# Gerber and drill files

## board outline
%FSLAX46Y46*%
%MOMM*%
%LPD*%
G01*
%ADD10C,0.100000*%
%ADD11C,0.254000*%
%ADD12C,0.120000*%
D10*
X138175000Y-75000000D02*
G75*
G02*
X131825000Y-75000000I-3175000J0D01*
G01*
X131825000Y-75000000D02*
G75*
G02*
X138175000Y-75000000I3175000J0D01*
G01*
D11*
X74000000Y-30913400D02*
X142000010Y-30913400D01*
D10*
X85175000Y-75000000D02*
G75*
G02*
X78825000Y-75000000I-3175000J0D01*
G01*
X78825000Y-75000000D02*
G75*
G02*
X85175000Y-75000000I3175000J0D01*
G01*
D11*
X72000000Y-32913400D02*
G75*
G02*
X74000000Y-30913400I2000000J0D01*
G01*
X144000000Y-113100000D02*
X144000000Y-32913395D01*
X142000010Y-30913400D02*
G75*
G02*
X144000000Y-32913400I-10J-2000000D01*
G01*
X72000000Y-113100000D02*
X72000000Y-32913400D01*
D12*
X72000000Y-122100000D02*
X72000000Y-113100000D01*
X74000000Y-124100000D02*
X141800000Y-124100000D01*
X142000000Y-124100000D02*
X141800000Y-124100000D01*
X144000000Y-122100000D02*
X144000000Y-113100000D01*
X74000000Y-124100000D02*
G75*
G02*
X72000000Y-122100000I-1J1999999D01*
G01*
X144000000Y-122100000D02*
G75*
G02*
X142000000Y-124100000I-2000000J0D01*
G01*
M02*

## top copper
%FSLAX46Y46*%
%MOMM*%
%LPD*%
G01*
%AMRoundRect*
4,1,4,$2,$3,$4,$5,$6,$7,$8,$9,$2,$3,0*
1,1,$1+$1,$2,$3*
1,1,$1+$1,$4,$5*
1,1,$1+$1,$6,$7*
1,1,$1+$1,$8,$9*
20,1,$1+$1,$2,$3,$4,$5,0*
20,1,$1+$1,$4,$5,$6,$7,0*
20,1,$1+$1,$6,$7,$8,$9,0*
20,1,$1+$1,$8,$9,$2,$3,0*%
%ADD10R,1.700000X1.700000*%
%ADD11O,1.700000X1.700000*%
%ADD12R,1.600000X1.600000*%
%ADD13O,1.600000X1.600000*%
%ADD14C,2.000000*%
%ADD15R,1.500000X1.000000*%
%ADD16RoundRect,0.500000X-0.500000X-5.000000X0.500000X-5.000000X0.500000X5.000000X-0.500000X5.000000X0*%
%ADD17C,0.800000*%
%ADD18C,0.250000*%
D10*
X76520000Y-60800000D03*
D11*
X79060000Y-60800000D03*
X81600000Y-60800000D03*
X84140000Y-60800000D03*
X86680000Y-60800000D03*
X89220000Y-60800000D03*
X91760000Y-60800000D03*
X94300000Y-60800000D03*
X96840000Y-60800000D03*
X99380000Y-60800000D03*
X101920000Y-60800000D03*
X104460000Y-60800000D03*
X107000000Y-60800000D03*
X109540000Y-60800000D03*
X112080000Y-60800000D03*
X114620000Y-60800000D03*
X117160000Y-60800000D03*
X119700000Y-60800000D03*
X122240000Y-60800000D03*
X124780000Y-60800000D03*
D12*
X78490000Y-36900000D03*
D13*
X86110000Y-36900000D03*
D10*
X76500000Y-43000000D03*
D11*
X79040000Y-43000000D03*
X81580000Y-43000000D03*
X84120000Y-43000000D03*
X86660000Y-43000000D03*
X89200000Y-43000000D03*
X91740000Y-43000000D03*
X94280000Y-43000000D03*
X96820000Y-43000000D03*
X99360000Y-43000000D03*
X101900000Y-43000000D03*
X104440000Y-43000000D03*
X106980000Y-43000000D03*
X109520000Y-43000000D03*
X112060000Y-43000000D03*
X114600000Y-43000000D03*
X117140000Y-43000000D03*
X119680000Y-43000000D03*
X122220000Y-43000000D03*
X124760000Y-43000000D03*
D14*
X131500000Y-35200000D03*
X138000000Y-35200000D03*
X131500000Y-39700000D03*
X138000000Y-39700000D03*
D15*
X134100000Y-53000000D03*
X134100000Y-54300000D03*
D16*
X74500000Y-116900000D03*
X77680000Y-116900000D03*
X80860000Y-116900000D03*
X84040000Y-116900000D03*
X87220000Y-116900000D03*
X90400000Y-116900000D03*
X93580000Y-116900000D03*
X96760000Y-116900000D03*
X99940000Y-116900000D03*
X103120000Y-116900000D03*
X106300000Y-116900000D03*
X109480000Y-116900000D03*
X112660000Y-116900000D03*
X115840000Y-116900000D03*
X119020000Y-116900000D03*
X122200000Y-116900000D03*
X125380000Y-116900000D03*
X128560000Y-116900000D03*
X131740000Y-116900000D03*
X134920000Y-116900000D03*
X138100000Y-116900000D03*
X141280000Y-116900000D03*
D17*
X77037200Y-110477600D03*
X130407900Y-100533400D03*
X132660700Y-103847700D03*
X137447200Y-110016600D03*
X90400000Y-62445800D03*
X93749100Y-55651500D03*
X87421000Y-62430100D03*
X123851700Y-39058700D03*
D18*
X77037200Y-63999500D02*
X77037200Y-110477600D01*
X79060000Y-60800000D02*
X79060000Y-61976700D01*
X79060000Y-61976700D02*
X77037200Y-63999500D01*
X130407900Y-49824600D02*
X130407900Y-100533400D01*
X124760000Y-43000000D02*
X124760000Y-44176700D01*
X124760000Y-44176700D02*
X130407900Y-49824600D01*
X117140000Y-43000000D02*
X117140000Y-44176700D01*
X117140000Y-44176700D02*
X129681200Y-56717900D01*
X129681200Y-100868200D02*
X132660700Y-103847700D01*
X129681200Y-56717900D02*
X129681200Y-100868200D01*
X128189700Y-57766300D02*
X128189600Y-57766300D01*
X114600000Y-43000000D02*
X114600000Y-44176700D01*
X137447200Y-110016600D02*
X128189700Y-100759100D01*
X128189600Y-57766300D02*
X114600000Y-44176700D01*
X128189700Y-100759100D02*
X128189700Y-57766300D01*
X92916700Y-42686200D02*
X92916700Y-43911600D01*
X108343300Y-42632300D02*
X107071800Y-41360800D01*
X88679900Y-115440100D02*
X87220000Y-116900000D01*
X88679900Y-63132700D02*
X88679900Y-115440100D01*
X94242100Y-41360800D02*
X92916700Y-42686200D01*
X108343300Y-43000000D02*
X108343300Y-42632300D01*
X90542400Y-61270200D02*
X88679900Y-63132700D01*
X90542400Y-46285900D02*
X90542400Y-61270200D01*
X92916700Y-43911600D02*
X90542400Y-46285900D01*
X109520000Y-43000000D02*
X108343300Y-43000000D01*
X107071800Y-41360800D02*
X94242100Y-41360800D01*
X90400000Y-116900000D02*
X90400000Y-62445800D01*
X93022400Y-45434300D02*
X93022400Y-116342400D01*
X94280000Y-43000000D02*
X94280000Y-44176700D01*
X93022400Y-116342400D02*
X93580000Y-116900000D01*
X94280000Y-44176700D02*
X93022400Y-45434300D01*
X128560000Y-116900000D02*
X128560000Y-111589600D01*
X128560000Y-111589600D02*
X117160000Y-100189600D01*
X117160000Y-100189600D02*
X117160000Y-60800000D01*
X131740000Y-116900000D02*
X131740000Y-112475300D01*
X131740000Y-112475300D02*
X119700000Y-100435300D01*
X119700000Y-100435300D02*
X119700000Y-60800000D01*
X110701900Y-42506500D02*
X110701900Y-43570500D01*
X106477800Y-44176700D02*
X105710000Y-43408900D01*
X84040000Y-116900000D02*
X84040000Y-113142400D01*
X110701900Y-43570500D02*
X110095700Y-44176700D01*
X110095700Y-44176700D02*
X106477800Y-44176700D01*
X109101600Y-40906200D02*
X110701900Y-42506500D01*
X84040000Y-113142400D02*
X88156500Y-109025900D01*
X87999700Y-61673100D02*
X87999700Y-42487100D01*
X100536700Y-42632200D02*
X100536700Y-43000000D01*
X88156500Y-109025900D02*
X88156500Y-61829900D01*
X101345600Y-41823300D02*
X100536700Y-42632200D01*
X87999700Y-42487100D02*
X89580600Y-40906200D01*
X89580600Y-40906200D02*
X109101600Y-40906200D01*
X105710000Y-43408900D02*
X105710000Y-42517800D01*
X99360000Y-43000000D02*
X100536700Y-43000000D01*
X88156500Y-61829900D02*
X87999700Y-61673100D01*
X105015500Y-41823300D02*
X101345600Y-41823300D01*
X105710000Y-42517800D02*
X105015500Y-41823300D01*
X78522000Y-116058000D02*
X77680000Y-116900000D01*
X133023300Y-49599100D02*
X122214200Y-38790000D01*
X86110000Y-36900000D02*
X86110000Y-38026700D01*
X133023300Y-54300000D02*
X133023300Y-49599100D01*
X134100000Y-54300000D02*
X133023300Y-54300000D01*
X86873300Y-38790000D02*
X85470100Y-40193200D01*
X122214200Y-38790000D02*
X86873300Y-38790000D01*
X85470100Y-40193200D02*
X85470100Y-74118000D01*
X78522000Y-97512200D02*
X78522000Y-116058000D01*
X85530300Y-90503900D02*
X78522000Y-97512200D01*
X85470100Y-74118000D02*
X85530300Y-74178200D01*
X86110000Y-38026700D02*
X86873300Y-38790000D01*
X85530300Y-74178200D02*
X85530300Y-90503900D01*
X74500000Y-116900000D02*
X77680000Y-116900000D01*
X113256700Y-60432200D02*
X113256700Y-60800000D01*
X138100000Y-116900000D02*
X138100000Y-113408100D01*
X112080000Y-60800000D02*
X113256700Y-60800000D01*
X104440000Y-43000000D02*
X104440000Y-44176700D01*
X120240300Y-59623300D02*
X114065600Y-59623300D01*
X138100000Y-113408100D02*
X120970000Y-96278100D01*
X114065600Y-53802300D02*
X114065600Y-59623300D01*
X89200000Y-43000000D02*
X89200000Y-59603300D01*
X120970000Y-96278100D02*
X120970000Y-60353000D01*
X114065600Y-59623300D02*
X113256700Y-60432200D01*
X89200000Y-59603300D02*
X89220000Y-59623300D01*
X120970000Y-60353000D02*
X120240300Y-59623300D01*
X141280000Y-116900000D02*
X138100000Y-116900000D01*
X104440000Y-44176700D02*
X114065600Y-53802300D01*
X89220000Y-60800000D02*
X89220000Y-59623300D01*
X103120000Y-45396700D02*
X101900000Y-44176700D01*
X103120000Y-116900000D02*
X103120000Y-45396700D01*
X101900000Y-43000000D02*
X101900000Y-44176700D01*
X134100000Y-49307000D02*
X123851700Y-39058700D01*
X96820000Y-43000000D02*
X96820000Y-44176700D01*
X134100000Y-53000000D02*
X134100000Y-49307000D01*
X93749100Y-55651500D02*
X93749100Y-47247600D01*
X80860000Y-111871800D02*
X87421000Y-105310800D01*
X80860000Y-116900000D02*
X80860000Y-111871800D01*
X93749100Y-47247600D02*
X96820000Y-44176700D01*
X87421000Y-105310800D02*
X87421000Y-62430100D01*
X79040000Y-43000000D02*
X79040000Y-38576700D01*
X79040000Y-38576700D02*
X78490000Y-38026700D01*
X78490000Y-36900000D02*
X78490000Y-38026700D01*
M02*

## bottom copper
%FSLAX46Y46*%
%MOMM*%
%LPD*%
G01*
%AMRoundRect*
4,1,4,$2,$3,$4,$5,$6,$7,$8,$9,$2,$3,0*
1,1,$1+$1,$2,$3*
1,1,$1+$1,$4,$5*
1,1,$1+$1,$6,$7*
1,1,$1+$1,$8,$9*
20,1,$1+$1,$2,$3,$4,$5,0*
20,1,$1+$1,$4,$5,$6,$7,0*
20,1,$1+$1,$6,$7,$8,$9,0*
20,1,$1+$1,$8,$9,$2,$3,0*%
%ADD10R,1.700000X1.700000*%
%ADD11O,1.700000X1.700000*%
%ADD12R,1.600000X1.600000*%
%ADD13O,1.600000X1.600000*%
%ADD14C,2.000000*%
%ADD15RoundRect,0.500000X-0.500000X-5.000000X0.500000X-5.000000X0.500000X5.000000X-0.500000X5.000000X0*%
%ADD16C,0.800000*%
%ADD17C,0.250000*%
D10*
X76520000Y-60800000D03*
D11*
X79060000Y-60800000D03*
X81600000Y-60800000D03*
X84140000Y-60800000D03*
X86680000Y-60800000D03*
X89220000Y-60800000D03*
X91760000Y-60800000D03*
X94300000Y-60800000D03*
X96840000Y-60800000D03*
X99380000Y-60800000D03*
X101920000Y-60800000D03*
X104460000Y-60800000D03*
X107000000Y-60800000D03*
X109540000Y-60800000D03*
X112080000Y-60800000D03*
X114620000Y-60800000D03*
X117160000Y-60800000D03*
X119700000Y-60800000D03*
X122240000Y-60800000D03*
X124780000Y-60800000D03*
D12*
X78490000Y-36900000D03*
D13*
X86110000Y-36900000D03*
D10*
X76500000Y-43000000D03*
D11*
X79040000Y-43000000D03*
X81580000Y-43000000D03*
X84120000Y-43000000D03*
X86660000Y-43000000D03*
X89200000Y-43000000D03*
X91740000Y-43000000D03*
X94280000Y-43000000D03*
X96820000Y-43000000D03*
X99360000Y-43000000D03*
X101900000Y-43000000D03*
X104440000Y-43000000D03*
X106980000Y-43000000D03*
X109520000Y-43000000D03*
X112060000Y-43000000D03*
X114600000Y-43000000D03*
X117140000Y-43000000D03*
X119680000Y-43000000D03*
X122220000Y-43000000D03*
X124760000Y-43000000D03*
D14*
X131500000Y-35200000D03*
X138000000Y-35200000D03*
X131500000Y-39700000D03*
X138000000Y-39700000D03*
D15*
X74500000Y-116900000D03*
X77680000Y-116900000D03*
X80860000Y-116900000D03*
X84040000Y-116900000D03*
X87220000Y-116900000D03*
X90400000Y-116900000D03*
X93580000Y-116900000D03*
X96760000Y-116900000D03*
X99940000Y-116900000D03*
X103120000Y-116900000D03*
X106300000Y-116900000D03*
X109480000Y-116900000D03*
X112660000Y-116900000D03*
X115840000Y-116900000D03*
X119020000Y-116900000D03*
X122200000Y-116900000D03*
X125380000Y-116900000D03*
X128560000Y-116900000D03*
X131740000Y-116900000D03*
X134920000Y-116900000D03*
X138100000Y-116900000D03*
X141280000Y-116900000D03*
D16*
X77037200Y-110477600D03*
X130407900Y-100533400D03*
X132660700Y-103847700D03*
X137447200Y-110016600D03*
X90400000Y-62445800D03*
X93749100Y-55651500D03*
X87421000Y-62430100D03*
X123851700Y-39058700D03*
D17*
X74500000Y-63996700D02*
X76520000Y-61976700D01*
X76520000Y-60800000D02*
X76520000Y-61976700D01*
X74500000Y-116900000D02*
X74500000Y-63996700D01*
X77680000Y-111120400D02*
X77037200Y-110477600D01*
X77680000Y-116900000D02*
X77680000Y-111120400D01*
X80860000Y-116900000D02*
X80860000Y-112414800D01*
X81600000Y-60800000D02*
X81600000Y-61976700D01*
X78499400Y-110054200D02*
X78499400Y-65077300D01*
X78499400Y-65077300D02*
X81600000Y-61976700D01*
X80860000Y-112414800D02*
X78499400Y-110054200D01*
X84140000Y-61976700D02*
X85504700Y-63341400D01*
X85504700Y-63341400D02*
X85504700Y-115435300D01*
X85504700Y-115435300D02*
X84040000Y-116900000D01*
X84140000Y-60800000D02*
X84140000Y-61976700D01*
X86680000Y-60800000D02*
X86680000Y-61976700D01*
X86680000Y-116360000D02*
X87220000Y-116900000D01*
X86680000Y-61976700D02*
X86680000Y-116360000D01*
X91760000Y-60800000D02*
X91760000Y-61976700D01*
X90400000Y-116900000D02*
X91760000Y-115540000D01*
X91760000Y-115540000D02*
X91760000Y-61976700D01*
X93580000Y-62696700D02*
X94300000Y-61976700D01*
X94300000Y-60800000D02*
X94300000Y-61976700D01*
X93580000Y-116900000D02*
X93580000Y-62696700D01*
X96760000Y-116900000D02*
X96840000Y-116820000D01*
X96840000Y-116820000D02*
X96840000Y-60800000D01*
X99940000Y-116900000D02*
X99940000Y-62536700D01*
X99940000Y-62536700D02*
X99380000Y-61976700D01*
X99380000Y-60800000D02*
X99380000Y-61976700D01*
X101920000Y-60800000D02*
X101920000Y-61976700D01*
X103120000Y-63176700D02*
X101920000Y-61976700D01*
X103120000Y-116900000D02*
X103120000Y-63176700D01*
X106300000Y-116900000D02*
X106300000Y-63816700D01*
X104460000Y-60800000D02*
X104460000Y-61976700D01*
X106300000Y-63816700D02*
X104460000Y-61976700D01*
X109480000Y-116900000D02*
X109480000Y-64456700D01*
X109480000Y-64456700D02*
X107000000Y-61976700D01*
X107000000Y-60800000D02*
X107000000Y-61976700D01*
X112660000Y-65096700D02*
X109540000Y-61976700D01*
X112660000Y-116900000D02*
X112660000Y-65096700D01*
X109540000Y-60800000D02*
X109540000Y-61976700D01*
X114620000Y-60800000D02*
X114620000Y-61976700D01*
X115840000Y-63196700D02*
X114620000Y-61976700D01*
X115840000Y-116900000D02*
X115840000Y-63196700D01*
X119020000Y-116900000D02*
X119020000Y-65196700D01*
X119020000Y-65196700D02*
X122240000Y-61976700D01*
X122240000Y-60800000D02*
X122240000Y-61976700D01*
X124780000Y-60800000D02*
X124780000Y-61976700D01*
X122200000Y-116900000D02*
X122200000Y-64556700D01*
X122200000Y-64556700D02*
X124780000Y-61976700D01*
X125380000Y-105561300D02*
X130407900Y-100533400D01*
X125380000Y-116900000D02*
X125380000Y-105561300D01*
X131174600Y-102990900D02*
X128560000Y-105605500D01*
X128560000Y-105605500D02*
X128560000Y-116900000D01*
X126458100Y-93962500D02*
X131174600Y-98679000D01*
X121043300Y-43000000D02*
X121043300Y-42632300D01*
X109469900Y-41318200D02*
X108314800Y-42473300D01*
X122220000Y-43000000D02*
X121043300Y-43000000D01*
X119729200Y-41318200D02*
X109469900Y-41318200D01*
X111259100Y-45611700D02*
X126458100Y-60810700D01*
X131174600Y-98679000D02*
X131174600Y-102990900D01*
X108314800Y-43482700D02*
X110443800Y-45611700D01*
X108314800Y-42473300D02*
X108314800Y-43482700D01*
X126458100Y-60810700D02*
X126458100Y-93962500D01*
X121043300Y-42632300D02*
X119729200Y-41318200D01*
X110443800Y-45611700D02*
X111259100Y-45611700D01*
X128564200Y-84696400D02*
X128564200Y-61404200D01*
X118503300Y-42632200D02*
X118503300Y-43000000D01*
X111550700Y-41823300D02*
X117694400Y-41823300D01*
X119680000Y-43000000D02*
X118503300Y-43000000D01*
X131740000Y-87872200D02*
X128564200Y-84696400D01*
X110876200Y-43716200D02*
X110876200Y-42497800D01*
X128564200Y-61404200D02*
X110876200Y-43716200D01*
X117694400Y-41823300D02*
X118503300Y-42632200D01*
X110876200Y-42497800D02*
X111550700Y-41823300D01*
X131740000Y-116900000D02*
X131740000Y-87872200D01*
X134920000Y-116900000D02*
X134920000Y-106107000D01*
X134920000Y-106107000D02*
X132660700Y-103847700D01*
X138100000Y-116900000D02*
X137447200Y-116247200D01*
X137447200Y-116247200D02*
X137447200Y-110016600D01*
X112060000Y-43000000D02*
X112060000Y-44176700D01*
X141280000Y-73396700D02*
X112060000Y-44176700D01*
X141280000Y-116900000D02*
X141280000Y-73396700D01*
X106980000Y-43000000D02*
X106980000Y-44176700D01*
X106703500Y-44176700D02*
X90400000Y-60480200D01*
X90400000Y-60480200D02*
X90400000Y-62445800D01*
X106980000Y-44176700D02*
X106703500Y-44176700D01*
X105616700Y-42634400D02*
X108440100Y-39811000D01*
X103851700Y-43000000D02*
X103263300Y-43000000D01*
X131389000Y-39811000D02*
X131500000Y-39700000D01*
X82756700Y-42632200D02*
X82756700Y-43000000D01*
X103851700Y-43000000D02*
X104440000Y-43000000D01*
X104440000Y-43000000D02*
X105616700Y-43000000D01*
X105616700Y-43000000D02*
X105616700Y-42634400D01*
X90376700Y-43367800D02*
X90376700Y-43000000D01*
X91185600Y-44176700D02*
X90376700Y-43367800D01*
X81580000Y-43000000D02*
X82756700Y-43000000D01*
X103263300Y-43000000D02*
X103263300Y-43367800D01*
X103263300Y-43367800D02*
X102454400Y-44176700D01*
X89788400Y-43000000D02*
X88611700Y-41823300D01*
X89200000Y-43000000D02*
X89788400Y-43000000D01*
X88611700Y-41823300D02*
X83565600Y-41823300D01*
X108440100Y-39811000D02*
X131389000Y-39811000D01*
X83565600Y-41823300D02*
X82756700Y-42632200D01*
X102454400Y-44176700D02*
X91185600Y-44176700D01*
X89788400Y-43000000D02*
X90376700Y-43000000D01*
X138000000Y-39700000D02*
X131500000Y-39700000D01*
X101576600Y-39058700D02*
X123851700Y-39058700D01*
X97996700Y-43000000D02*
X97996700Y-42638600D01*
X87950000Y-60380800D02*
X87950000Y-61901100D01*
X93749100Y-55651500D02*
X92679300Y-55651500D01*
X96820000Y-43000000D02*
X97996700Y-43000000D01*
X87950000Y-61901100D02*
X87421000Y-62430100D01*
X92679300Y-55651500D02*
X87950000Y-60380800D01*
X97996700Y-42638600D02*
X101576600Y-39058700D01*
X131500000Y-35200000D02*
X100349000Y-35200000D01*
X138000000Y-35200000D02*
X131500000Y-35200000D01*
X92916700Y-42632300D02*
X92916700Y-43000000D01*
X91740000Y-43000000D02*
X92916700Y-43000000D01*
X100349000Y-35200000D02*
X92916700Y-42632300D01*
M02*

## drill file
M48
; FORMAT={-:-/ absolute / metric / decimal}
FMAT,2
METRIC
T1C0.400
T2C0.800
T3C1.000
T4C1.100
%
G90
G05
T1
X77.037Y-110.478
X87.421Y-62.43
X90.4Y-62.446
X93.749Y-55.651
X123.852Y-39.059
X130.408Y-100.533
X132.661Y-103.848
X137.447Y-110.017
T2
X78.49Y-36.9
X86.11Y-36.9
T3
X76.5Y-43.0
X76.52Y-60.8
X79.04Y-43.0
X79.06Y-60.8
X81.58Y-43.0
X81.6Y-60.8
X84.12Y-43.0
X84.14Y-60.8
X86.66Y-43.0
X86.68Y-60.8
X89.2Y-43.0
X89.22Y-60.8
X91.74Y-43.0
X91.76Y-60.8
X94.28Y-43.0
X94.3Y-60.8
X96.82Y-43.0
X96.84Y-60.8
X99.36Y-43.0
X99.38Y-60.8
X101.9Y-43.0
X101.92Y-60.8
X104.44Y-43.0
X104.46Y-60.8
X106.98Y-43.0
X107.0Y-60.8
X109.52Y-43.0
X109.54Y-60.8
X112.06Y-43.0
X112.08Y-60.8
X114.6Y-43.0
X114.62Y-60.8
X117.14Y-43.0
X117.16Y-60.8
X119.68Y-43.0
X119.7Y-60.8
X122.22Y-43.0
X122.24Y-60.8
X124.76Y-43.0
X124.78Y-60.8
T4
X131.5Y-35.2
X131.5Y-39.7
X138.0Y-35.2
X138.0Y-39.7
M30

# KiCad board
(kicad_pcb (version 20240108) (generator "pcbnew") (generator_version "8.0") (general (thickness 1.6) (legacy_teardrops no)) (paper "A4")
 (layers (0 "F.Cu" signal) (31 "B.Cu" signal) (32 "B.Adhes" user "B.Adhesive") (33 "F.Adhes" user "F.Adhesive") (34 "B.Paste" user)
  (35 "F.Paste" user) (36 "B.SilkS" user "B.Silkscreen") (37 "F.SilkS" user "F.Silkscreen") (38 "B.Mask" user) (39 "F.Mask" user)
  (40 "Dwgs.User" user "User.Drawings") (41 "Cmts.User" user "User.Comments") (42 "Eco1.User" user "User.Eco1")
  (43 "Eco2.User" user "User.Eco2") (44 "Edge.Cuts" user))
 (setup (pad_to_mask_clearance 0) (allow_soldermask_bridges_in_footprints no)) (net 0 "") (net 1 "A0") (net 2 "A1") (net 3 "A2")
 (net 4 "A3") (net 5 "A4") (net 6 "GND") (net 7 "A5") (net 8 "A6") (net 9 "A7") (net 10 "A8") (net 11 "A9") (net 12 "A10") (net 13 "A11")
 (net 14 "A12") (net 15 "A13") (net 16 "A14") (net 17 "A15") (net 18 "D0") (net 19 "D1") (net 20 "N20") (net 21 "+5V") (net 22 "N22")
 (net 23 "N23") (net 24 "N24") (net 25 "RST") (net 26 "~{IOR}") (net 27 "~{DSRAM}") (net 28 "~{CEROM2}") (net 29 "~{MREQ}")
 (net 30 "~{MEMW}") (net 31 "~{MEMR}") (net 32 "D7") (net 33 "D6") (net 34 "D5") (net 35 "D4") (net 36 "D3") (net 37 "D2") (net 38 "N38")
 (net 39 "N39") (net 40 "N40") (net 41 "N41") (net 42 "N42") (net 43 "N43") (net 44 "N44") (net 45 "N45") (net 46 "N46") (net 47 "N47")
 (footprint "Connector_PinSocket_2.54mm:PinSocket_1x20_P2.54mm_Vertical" (layer "F.Cu") (at 76.52 60.8 90)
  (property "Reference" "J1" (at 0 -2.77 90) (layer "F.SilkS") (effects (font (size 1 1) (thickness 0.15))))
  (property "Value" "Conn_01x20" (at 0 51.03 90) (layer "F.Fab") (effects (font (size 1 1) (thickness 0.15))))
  (pad "1" thru_hole rect (at 0 0 90) (size 1.7 1.7) (drill 1) (layers "*.Cu" "*.Mask") (remove_unused_layers no) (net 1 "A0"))
  (pad "2" thru_hole oval (at 0 2.54 90) (size 1.7 1.7) (drill 1) (layers "*.Cu" "*.Mask") (remove_unused_layers no) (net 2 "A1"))
  (pad "3" thru_hole oval (at 0 5.08 90) (size 1.7 1.7) (drill 1) (layers "*.Cu" "*.Mask") (remove_unused_layers no) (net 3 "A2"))
  (pad "4" thru_hole oval (at 0 7.62 90) (size 1.7 1.7) (drill 1) (layers "*.Cu" "*.Mask") (remove_unused_layers no) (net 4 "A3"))
  (pad "5" thru_hole oval (at 0 10.16 90) (size 1.7 1.7) (drill 1) (layers "*.Cu" "*.Mask") (remove_unused_layers no) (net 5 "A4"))
  (pad "6" thru_hole oval (at 0 12.7 90) (size 1.7 1.7) (drill 1) (layers "*.Cu" "*.Mask") (remove_unused_layers no) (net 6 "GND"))
  (pad "7" thru_hole oval (at 0 15.24 90) (size 1.7 1.7) (drill 1) (layers "*.Cu" "*.Mask") (remove_unused_layers no) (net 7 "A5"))
  (pad "8" thru_hole oval (at 0 17.78 90) (size 1.7 1.7) (drill 1) (layers "*.Cu" "*.Mask") (remove_unused_layers no) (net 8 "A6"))
  (pad "9" thru_hole oval (at 0 20.32 90) (size 1.7 1.7) (drill 1) (layers "*.Cu" "*.Mask") (remove_unused_layers no) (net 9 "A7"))
  (pad "10" thru_hole oval (at 0 22.86 90) (size 1.7 1.7) (drill 1) (layers "*.Cu" "*.Mask") (remove_unused_layers no) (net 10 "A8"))
  (pad "11" thru_hole oval (at 0 25.4 90) (size 1.7 1.7) (drill 1) (layers "*.Cu" "*.Mask") (remove_unused_layers no) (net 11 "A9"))
  (pad "12" thru_hole oval (at 0 27.94 90) (size 1.7 1.7) (drill 1) (layers "*.Cu" "*.Mask") (remove_unused_layers no) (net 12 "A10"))
  (pad "13" thru_hole oval (at 0 30.48 90) (size 1.7 1.7) (drill 1) (layers "*.Cu" "*.Mask") (remove_unused_layers no) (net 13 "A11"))
  (pad "14" thru_hole oval (at 0 33.02 90) (size 1.7 1.7) (drill 1) (layers "*.Cu" "*.Mask") (remove_unused_layers no) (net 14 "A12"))
  (pad "15" thru_hole oval (at 0 35.56 90) (size 1.7 1.7) (drill 1) (layers "*.Cu" "*.Mask") (remove_unused_layers no) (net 6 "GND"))
  (pad "16" thru_hole oval (at 0 38.1 90) (size 1.7 1.7) (drill 1) (layers "*.Cu" "*.Mask") (remove_unused_layers no) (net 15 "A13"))
  (pad "17" thru_hole oval (at 0 40.64 90) (size 1.7 1.7) (drill 1) (layers "*.Cu" "*.Mask") (remove_unused_layers no) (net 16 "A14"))
  (pad "18" thru_hole oval (at 0 43.18 90) (size 1.7 1.7) (drill 1) (layers "*.Cu" "*.Mask") (remove_unused_layers no) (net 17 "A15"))
  (pad "19" thru_hole oval (at 0 45.72 90) (size 1.7 1.7) (drill 1) (layers "*.Cu" "*.Mask") (remove_unused_layers no) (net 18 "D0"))
  (pad "20" thru_hole oval (at 0 48.26 90) (size 1.7 1.7) (drill 1) (layers "*.Cu" "*.Mask") (remove_unused_layers no) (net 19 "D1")))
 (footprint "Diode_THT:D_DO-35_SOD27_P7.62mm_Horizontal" (layer "F.Cu") (at 78.49 36.9)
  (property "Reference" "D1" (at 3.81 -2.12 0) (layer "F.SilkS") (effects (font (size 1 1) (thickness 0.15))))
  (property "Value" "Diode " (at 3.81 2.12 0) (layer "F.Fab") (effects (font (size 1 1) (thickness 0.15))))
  (pad "1" thru_hole rect (at 0 0) (size 1.6 1.6) (drill 0.8) (layers "*.Cu" "*.Mask") (remove_unused_layers no) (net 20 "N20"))
  (pad "2" thru_hole oval (at 7.62 0) (size 1.6 1.6) (drill 0.8) (layers "*.Cu" "*.Mask") (remove_unused_layers no) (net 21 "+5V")))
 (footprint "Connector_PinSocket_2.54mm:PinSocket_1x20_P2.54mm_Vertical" (layer "F.Cu") (at 76.5 43 90)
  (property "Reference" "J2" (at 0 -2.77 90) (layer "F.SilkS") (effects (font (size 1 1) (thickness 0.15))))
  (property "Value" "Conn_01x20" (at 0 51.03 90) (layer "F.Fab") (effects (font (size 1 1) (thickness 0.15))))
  (pad "1" thru_hole rect (at 0 0 90) (size 1.7 1.7) (drill 1) (layers "*.Cu" "*.Mask") (remove_unused_layers no) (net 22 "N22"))
  (pad "2" thru_hole oval (at 0 2.54 90) (size 1.7 1.7) (drill 1) (layers "*.Cu" "*.Mask") (remove_unused_layers no) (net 20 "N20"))
  (pad "3" thru_hole oval (at 0 5.08 90) (size 1.7 1.7) (drill 1) (layers "*.Cu" "*.Mask") (remove_unused_layers no) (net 6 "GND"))
  (pad "4" thru_hole oval (at 0 7.62 90) (size 1.7 1.7) (drill 1) (layers "*.Cu" "*.Mask") (remove_unused_layers no) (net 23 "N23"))
  (pad "5" thru_hole oval (at 0 10.16 90) (size 1.7 1.7) (drill 1) (layers "*.Cu" "*.Mask") (remove_unused_layers no) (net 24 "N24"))
  (pad "6" thru_hole oval (at 0 12.7 90) (size 1.7 1.7) (drill 1) (layers "*.Cu" "*.Mask") (remove_unused_layers no) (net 6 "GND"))
  (pad "7" thru_hole oval (at 0 15.24 90) (size 1.7 1.7) (drill 1) (layers "*.Cu" "*.Mask") (remove_unused_layers no) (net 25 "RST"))
  (pad "8" thru_hole oval (at 0 17.78 90) (size 1.7 1.7) (drill 1) (layers "*.Cu" "*.Mask") (remove_unused_layers no) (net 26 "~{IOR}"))
  (pad "9" thru_hole oval (at 0 20.32 90) (size 1.7 1.7) (drill 1) (layers "*.Cu" "*.Mask") (remove_unused_layers no) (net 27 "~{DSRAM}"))
  (pad "10" thru_hole oval (at 0 22.86 90) (size 1.7 1.7) (drill 1) (layers "*.Cu" "*.Mask") (remove_unused_layers no) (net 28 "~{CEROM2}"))
  (pad "11" thru_hole oval (at 0 25.4 90) (size 1.7 1.7) (drill 1) (layers "*.Cu" "*.Mask") (remove_unused_layers no) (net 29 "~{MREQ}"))
  (pad "12" thru_hole oval (at 0 27.94 90) (size 1.7 1.7) (drill 1) (layers "*.Cu" "*.Mask") (remove_unused_layers no) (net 6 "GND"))
  (pad "13" thru_hole oval (at 0 30.48 90) (size 1.7 1.7) (drill 1) (layers "*.Cu" "*.Mask") (remove_unused_layers no) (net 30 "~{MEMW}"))
  (pad "14" thru_hole oval (at 0 33.02 90) (size 1.7 1.7) (drill 1) (layers "*.Cu" "*.Mask") (remove_unused_layers no) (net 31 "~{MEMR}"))
  (pad "15" thru_hole oval (at 0 35.56 90) (size 1.7 1.7) (drill 1) (layers "*.Cu" "*.Mask") (remove_unused_layers no) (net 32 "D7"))
  (pad "16" thru_hole oval (at 0 38.1 90) (size 1.7 1.7) (drill 1) (layers "*.Cu" "*.Mask") (remove_unused_layers no) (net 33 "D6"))
  (pad "17" thru_hole oval (at 0 40.64 90) (size 1.7 1.7) (drill 1) (layers "*.Cu" "*.Mask") (remove_unused_layers no) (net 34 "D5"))
  (pad "18" thru_hole oval (at 0 43.18 90) (size 1.7 1.7) (drill 1) (layers "*.Cu" "*.Mask") (remove_unused_layers no) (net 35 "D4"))
  (pad "19" thru_hole oval (at 0 45.72 90) (size 1.7 1.7) (drill 1) (layers "*.Cu" "*.Mask") (remove_unused_layers no) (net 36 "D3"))
  (pad "20" thru_hole oval (at 0 48.26 90) (size 1.7 1.7) (drill 1) (layers "*.Cu" "*.Mask") (remove_unused_layers no) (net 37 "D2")))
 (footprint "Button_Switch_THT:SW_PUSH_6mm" (layer "F.Cu") (at 131.5 35.2)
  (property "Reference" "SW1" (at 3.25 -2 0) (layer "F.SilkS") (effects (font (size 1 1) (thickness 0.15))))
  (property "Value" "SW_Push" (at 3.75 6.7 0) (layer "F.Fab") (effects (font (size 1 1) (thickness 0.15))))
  (pad "1" thru_hole circle (at 0 0 90) (size 2 2) (drill 1.1) (layers "*.Cu" "*.Mask") (remove_unused_layers no) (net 25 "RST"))
  (pad "1" thru_hole circle (at 6.5 0 90) (size 2 2) (drill 1.1) (layers "*.Cu" "*.Mask") (remove_unused_layers no) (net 25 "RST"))
  (pad "2" thru_hole circle (at 0 4.5 90) (size 2 2) (drill 1.1) (layers "*.Cu" "*.Mask") (remove_unused_layers no) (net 6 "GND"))
  (pad "2" thru_hole circle (at 6.5 4.5 90) (size 2 2) (drill 1.1) (layers "*.Cu" "*.Mask") (remove_unused_layers no) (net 6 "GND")))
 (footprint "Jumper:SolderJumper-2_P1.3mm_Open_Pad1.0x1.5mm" (layer "F.Cu") (at 134.1 53.65 -90)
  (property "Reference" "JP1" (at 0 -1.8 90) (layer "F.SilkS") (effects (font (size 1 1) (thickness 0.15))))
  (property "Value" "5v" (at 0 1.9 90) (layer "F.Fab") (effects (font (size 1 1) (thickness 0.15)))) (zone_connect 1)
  (pad "1" smd rect (at -0.65 0 270) (size 1 1.5) (layers "F.Cu" "F.Mask") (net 27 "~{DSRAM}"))
  (pad "2" smd rect (at 0.65 0 270) (size 1 1.5) (layers "F.Cu" "F.Mask") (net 21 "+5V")))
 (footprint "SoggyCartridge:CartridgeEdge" (layer "F.Cu") (at 74.9 111.4)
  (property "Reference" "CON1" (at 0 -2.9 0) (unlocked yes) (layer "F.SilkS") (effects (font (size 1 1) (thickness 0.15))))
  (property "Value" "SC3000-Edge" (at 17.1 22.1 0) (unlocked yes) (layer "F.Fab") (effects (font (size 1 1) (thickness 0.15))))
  (fp_line (start -2.9 10.7) (end -2.9 1.7) (stroke (width 0.12) (type solid)) (layer "Edge.Cuts"))
  (fp_line (start -0.9 12.7) (end 66.9 12.7) (stroke (width 0.12) (type solid)) (layer "Edge.Cuts"))
  (fp_line (start 67.1 12.7) (end 66.9 12.7) (stroke (width 0.12) (type solid)) (layer "Edge.Cuts"))
  (fp_line (start 69.1 10.7) (end 69.1 1.7) (stroke (width 0.12) (type solid)) (layer "Edge.Cuts"))
  (fp_arc (start -0.9 12.7) (mid -2.314214 12.114214) (end -2.9 10.7) (stroke (width 0.12) (type solid)) (layer "Edge.Cuts"))
  (fp_arc (start 69.1 10.7) (mid 68.514214 12.114214) (end 67.1 12.7) (stroke (width 0.12) (type solid)) (layer "Edge.Cuts"))
  (pad "A1" connect roundrect (at -0.4 5.5) (size 2 11) (layers "B.Cu" "B.Mask") (roundrect_rratio 0.25) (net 1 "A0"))
  (pad "A2" connect roundrect (at 2.78 5.5) (size 2 11) (layers "B.Cu" "B.Mask") (roundrect_rratio 0.25) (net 2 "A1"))
  (pad "A3" connect roundrect (at 5.96 5.5) (size 2 11) (layers "B.Cu" "B.Mask") (roundrect_rratio 0.25) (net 3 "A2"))
  (pad "A4" connect roundrect (at 9.14 5.5) (size 2 11) (layers "B.Cu" "B.Mask") (roundrect_rratio 0.25) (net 4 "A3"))
  (pad "A5" connect roundrect (at 12.32 5.5) (size 2 11) (layers "B.Cu" "B.Mask") (roundrect_rratio 0.25) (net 5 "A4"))
  (pad "A6" connect roundrect (at 15.5 5.5) (size 2 11) (layers "B.Cu" "B.Mask") (roundrect_rratio 0.25) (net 7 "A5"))
  (pad "A7" connect roundrect (at 18.68 5.5) (size 2 11) (layers "B.Cu" "B.Mask") (roundrect_rratio 0.25) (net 8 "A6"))
  (pad "A8" connect roundrect (at 21.86 5.5) (size 2 11) (layers "B.Cu" "B.Mask") (roundrect_rratio 0.25) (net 9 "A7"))
  (pad "A9" connect roundrect (at 25.04 5.5) (size 2 11) (layers "B.Cu" "B.Mask") (roundrect_rratio 0.25) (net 10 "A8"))
  (pad "A10" connect roundrect (at 28.22 5.5) (size 2 11) (layers "B.Cu" "B.Mask") (roundrect_rratio 0.25) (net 11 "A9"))
  (pad "A11" connect roundrect (at 31.4 5.5) (size 2 11) (layers "B.Cu" "B.Mask") (roundrect_rratio 0.25) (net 12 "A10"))
  (pad "A12" connect roundrect (at 34.58 5.5) (size 2 11) (layers "B.Cu" "B.Mask") (roundrect_rratio 0.25) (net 13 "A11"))
  (pad "A13" connect roundrect (at 37.76 5.5) (size 2 11) (layers "B.Cu" "B.Mask") (roundrect_rratio 0.25) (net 14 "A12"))
  (pad "A14" connect roundrect (at 40.94 5.5) (size 2 11) (layers "B.Cu" "B.Mask") (roundrect_rratio 0.25) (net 15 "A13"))
  (pad "A15" connect roundrect (at 44.12 5.5) (size 2 11) (layers "B.Cu" "B.Mask") (roundrect_rratio 0.25) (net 18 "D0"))
  (pad "A16" connect roundrect (at 47.3 5.5) (size 2 11) (layers "B.Cu" "B.Mask") (roundrect_rratio 0.25) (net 19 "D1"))
  (pad "A17" connect roundrect (at 50.48 5.5) (size 2 11) (layers "B.Cu" "B.Mask") (roundrect_rratio 0.25) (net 37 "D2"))
  (pad "A18" connect roundrect (at 53.66 5.5) (size 2 11) (layers "B.Cu" "B.Mask") (roundrect_rratio 0.25) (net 36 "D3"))
  (pad "A19" connect roundrect (at 56.84 5.5) (size 2 11) (layers "B.Cu" "B.Mask") (roundrect_rratio 0.25) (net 35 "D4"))
  (pad "A20" connect roundrect (at 60.02 5.5) (size 2 11) (layers "B.Cu" "B.Mask") (roundrect_rratio 0.25) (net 34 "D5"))
  (pad "A21" connect roundrect (at 63.2 5.5) (size 2 11) (layers "B.Cu" "B.Mask") (roundrect_rratio 0.25) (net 33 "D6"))
  (pad "A22" connect roundrect (at 66.38 5.5) (size 2 11) (layers "B.Cu" "B.Mask") (roundrect_rratio 0.25) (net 32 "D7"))
  (pad "B1" connect roundrect (at -0.4 5.5) (size 2 11) (layers "F.Cu" "F.Mask") (roundrect_rratio 0.25) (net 21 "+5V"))
  (pad "B2" connect roundrect (at 2.78 5.5) (size 2 11) (layers "F.Cu" "F.Mask") (roundrect_rratio 0.25) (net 21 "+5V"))
  (pad "B3" connect roundrect (at 5.96 5.5) (size 2 11) (layers "F.Cu" "F.Mask") (roundrect_rratio 0.25) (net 27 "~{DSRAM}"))
  (pad "B4" connect roundrect (at 9.14 5.5) (size 2 11) (layers "F.Cu" "F.Mask") (roundrect_rratio 0.25) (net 28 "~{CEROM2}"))
  (pad "B5" connect roundrect (at 12.32 5.5) (size 2 11) (layers "F.Cu" "F.Mask") (roundrect_rratio 0.25) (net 31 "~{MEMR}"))
  (pad "B6" connect roundrect (at 15.5 5.5) (size 2 11) (layers "F.Cu" "F.Mask") (roundrect_rratio 0.25) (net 30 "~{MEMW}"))
  (pad "B7" connect roundrect (at 18.68 5.5) (size 2 11) (layers "F.Cu" "F.Mask") (roundrect_rratio 0.25) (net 26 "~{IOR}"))
  (pad "B8" connect roundrect (at 21.86 5.5) (size 2 11) (layers "F.Cu" "F.Mask") (roundrect_rratio 0.25) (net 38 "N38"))
  (pad "B9" connect roundrect (at 25.04 5.5) (size 2 11) (layers "F.Cu" "F.Mask") (roundrect_rratio 0.25) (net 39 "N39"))
  (pad "B10" connect roundrect (at 28.22 5.5) (size 2 11) (layers "F.Cu" "F.Mask") (roundrect_rratio 0.25) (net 29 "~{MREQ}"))
  (pad "B11" connect roundrect (at 31.4 5.5) (size 2 11) (layers "F.Cu" "F.Mask") (roundrect_rratio 0.25) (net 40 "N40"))
  (pad "B12" connect roundrect (at 34.58 5.5) (size 2 11) (layers "F.Cu" "F.Mask") (roundrect_rratio 0.25) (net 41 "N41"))
  (pad "B13" connect roundrect (at 37.76 5.5) (size 2 11) (layers "F.Cu" "F.Mask") (roundrect_rratio 0.25) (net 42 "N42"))
  (pad "B14" connect roundrect (at 40.94 5.5) (size 2 11) (layers "F.Cu" "F.Mask") (roundrect_rratio 0.25) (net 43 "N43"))
  (pad "B15" connect roundrect (at 44.12 5.5) (size 2 11) (layers "F.Cu" "F.Mask") (roundrect_rratio 0.25) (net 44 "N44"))
  (pad "B16" connect roundrect (at 47.3 5.5) (size 2 11) (layers "F.Cu" "F.Mask") (roundrect_rratio 0.25) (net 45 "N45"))
  (pad "B17" connect roundrect (at 50.48 5.5) (size 2 11) (layers "F.Cu" "F.Mask") (roundrect_rratio 0.25) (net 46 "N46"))
  (pad "B18" connect roundrect (at 53.66 5.5) (size 2 11) (layers "F.Cu" "F.Mask") (roundrect_rratio 0.25) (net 16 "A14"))
  (pad "B19" connect roundrect (at 56.84 5.5) (size 2 11) (layers "F.Cu" "F.Mask") (roundrect_rratio 0.25) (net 17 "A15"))
  (pad "B20" connect roundrect (at 60.02 5.5) (size 2 11) (layers "F.Cu" "F.Mask") (roundrect_rratio 0.25) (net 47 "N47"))
  (pad "B21" connect roundrect (at 63.2 5.5) (size 2 11) (layers "F.Cu" "F.Mask") (roundrect_rratio 0.25) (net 6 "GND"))
  (pad "B22" connect roundrect (at 66.38 5.5) (size 2 11) (layers "F.Cu" "F.Mask") (roundrect_rratio 0.25) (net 6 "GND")))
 (gr_circle (center 135 75) (end 138.175 75) (stroke (width 0.1) (type solid)) (fill none) (layer "Edge.Cuts"))
 (gr_line (start 74 30.9134) (end 142.00001 30.9134) (stroke (width 0.254) (type solid)) (layer "Edge.Cuts"))
 (gr_circle (center 82 75) (end 85.175 75) (stroke (width 0.1) (type solid)) (fill none) (layer "Edge.Cuts"))
 (gr_arc (start 72 32.9134) (mid 72.585786 31.499186) (end 74 30.9134) (stroke (width 0.254) (type solid)) (layer "Edge.Cuts"))
 (gr_line (start 144 113.1) (end 144 32.913395) (stroke (width 0.254) (type solid)) (layer "Edge.Cuts"))
 (gr_arc (start 142.00001 30.9134) (mid 143.414217 31.49919) (end 144.00001 32.9134) (stroke (width 0.254) (type solid)) (layer "Edge.Cuts"))
 (gr_line (start 72 113.1) (end 72 32.9134) (stroke (width 0.254) (type solid)) (layer "Edge.Cuts"))
 (segment (start 74.5 63.9967) (end 76.52 61.9767) (width 0.25) (layer "B.Cu") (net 1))
 (segment (start 76.52 60.8) (end 76.52 61.9767) (width 0.25) (layer "B.Cu") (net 1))
 (segment (start 74.5 116.9) (end 74.5 63.9967) (width 0.25) (layer "B.Cu") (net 1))
 (segment (start 77.0372 63.9995) (end 77.0372 110.4776) (width 0.25) (layer "F.Cu") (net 2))
 (segment (start 79.06 60.8) (end 79.06 61.9767) (width 0.25) (layer "F.Cu") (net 2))
 (segment (start 79.06 61.9767) (end 77.0372 63.9995) (width 0.25) (layer "F.Cu") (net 2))
 (via (at 77.0372 110.4776) (size 0.8) (drill 0.4) (layers "F.Cu" "B.Cu") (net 2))
 (segment (start 77.68 111.1204) (end 77.0372 110.4776) (width 0.25) (layer "B.Cu") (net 2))
 (segment (start 77.68 116.9) (end 77.68 111.1204) (width 0.25) (layer "B.Cu") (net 2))
 (segment (start 80.86 116.9) (end 80.86 112.4148) (width 0.25) (layer "B.Cu") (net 3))
 (segment (start 81.6 60.8) (end 81.6 61.9767) (width 0.25) (layer "B.Cu") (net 3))
 (segment (start 78.4994 110.0542) (end 78.4994 65.0773) (width 0.25) (layer "B.Cu") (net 3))
 (segment (start 78.4994 65.0773) (end 81.6 61.9767) (width 0.25) (layer "B.Cu") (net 3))
 (segment (start 80.86 112.4148) (end 78.4994 110.0542) (width 0.25) (layer "B.Cu") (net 3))
 (segment (start 84.14 61.9767) (end 85.5047 63.3414) (width 0.25) (layer "B.Cu") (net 4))
 (segment (start 85.5047 63.3414) (end 85.5047 115.4353) (width 0.25) (layer "B.Cu") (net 4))
 (segment (start 85.5047 115.4353) (end 84.04 116.9) (width 0.25) (layer "B.Cu") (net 4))
 (segment (start 84.14 60.8) (end 84.14 61.9767) (width 0.25) (layer "B.Cu") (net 4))
 (segment (start 86.68 60.8) (end 86.68 61.9767) (width 0.25) (layer "B.Cu") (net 5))
 (segment (start 86.68 116.36) (end 87.22 116.9) (width 0.25) (layer "B.Cu") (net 5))
 (segment (start 86.68 61.9767) (end 86.68 116.36) (width 0.25) (layer "B.Cu") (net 5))
 (segment (start 91.76 60.8) (end 91.76 61.9767) (width 0.25) (layer "B.Cu") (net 7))
 (segment (start 90.4 116.9) (end 91.76 115.54) (width 0.25) (layer "B.Cu") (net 7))
 (segment (start 91.76 115.54) (end 91.76 61.9767) (width 0.25) (layer "B.Cu") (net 7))
 (segment (start 93.58 62.6967) (end 94.3 61.9767) (width 0.25) (layer "B.Cu") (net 8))
 (segment (start 94.3 60.8) (end 94.3 61.9767) (width 0.25) (layer "B.Cu") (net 8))
 (segment (start 93.58 116.9) (end 93.58 62.6967) (width 0.25) (layer "B.Cu") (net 8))
 (segment (start 96.76 116.9) (end 96.84 116.82) (width 0.25) (layer "B.Cu") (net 9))
 (segment (start 96.84 116.82) (end 96.84 60.8) (width 0.25) (layer "B.Cu") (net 9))
 (segment (start 99.94 116.9) (end 99.94 62.5367) (width 0.25) (layer "B.Cu") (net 10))
 (segment (start 99.94 62.5367) (end 99.38 61.9767) (width 0.25) (layer "B.Cu") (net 10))
 (segment (start 99.38 60.8) (end 99.38 61.9767) (width 0.25) (layer "B.Cu") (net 10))
 (segment (start 101.92 60.8) (end 101.92 61.9767) (width 0.25) (layer "B.Cu") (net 11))
 (segment (start 103.12 63.1767) (end 101.92 61.9767) (width 0.25) (layer "B.Cu") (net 11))
 (segment (start 103.12 116.9) (end 103.12 63.1767) (width 0.25) (layer "B.Cu") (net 11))
 (segment (start 106.3 116.9) (end 106.3 63.8167) (width 0.25) (layer "B.Cu") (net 12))
 (segment (start 104.46 60.8) (end 104.46 61.9767) (width 0.25) (layer "B.Cu") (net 12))
 (segment (start 106.3 63.8167) (end 104.46 61.9767) (width 0.25) (layer "B.Cu") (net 12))
 (segment (start 109.48 116.9) (end 109.48 64.4567) (width 0.25) (layer "B.Cu") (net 13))
 (segment (start 109.48 64.4567) (end 107 61.9767) (width 0.25) (layer "B.Cu") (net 13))
 (segment (start 107 60.8) (end 107 61.9767) (width 0.25) (layer "B.Cu") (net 13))
 (segment (start 112.66 65.0967) (end 109.54 61.9767) (width 0.25) (layer "B.Cu") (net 14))
 (segment (start 112.66 116.9) (end 112.66 65.0967) (width 0.25) (layer "B.Cu") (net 14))
 (segment (start 109.54 60.8) (end 109.54 61.9767) (width 0.25) (layer "B.Cu") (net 14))
 (segment (start 114.62 60.8) (end 114.62 61.9767) (width 0.25) (layer "B.Cu") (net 15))
 (segment (start 115.84 63.1967) (end 114.62 61.9767) (width 0.25) (layer "B.Cu") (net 15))
 (segment (start 115.84 116.9) (end 115.84 63.1967) (width 0.25) (layer "B.Cu") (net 15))
 (segment (start 119.02 116.9) (end 119.02 65.1967) (width 0.25) (layer "B.Cu") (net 18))
 (segment (start 119.02 65.1967) (end 122.24 61.9767) (width 0.25) (layer "B.Cu") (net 18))
 (segment (start 122.24 60.8) (end 122.24 61.9767) (width 0.25) (layer "B.Cu") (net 18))
 (segment (start 124.78 60.8) (end 124.78 61.9767) (width 0.25) (layer "B.Cu") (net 19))
 (segment (start 122.2 116.9) (end 122.2 64.5567) (width 0.25) (layer "B.Cu") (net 19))
 (segment (start 122.2 64.5567) (end 124.78 61.9767) (width 0.25) (layer "B.Cu") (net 19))
 (segment (start 130.4079 49.8246) (end 130.4079 100.5334) (width 0.25) (layer "F.Cu") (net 37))
 (segment (start 124.76 43) (end 124.76 44.1767) (width 0.25) (layer "F.Cu") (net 37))
 (segment (start 124.76 44.1767) (end 130.4079 49.8246) (width 0.25) (layer "F.Cu") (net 37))
 (via (at 130.4079 100.5334) (size 0.8) (drill 0.4) (layers "F.Cu" "B.Cu") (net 37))
 (segment (start 125.38 105.5613) (end 130.4079 100.5334) (width 0.25) (layer "B.Cu") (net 37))
 (segment (start 125.38 116.9) (end 125.38 105.5613) (width 0.25) (layer "B.Cu") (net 37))
 (segment (start 131.1746 102.9909) (end 128.56 105.6055) (width 0.25) (layer "B.Cu") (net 36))
 (segment (start 128.56 105.6055) (end 128.56 116.9) (width 0.25) (layer "B.Cu") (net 36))
 (segment (start 126.4581 93.9625) (end 131.1746 98.679) (width 0.25) (layer "B.Cu") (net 36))
 (segment (start 121.0433 43) (end 121.0433 42.6323) (width 0.25) (layer "B.Cu") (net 36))
 (segment (start 109.4699 41.3182) (end 108.3148 42.4733) (width 0.25) (layer "B.Cu") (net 36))
 (segment (start 122.22 43) (end 121.0433 43) (width 0.25) (layer "B.Cu") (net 36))
 (segment (start 119.7292 41.3182) (end 109.4699 41.3182) (width 0.25) (layer "B.Cu") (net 36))
 (segment (start 111.2591 45.6117) (end 126.4581 60.8107) (width 0.25) (layer "B.Cu") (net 36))
 (segment (start 131.1746 98.679) (end 131.1746 102.9909) (width 0.25) (layer "B.Cu") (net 36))
 (segment (start 108.3148 43.4827) (end 110.4438 45.6117) (width 0.25) (layer "B.Cu") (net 36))
 (segment (start 108.3148 42.4733) (end 108.3148 43.4827) (width 0.25) (layer "B.Cu") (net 36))
 (segment (start 126.4581 60.8107) (end 126.4581 93.9625) (width 0.25) (layer "B.Cu") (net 36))
 (segment (start 121.0433 42.6323) (end 119.7292 41.3182) (width 0.25) (layer "B.Cu") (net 36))
 (segment (start 110.4438 45.6117) (end 111.2591 45.6117) (width 0.25) (layer "B.Cu") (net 36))
 (segment (start 128.5642 84.6964) (end 128.5642 61.4042) (width 0.25) (layer "B.Cu") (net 35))
 (segment (start 118.5033 42.6322) (end 118.5033 43) (width 0.25) (layer "B.Cu") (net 35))
 (segment (start 111.5507 41.8233) (end 117.6944 41.8233) (width 0.25) (layer "B.Cu") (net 35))
 (segment (start 119.68 43) (end 118.5033 43) (width 0.25) (layer "B.Cu") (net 35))
 (segment (start 131.74 87.8722) (end 128.5642 84.6964) (width 0.25) (layer "B.Cu") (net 35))
 (segment (start 110.8762 43.7162) (end 110.8762 42.4978) (width 0.25) (layer "B.Cu") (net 35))
 (segment (start 128.5642 61.4042) (end 110.8762 43.7162) (width 0.25) (layer "B.Cu") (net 35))
 (segment (start 117.6944 41.8233) (end 118.5033 42.6322) (width 0.25) (layer "B.Cu") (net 35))
 (segment (start 110.8762 42.4978) (end 111.5507 41.8233) (width 0.25) (layer "B.Cu") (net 35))
 (segment (start 131.74 116.9) (end 131.74 87.8722) (width 0.25) (layer "B.Cu") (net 35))
 (segment (start 117.14 43) (end 117.14 44.1767) (width 0.25) (layer "F.Cu") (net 34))
 (segment (start 117.14 44.1767) (end 129.6812 56.7179) (width 0.25) (layer "F.Cu") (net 34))
 (segment (start 129.6812 100.8682) (end 132.6607 103.8477) (width 0.25) (layer "F.Cu") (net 34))
 (segment (start 129.6812 56.7179) (end 129.6812 100.8682) (width 0.25) (layer "F.Cu") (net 34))
 (via (at 132.6607 103.8477) (size 0.8) (drill 0.4) (layers "F.Cu" "B.Cu") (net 34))
 (segment (start 134.92 116.9) (end 134.92 106.107) (width 0.25) (layer "B.Cu") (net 34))
 (segment (start 134.92 106.107) (end 132.6607 103.8477) (width 0.25) (layer "B.Cu") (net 34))
 (segment (start 128.1897 57.7663) (end 128.1896 57.7663) (width 0.25) (layer "F.Cu") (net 33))
 (segment (start 114.6 43) (end 114.6 44.1767) (width 0.25) (layer "F.Cu") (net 33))
 (segment (start 137.4472 110.0166) (end 128.1897 100.7591) (width 0.25) (layer "F.Cu") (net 33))
 (segment (start 128.1896 57.7663) (end 114.6 44.1767) (width 0.25) (layer "F.Cu") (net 33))
 (segment (start 128.1897 100.7591) (end 128.1897 57.7663) (width 0.25) (layer "F.Cu") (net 33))
 (via (at 137.4472 110.0166) (size 0.8) (drill 0.4) (layers "F.Cu" "B.Cu") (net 33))
 (segment (start 138.1 116.9) (end 137.4472 116.2472) (width 0.25) (layer "B.Cu") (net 33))
 (segment (start 137.4472 116.2472) (end 137.4472 110.0166) (width 0.25) (layer "B.Cu") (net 33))
 (segment (start 112.06 43) (end 112.06 44.1767) (width 0.25) (layer "B.Cu") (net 32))
 (segment (start 141.28 73.3967) (end 112.06 44.1767) (width 0.25) (layer "B.Cu") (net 32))
 (segment (start 141.28 116.9) (end 141.28 73.3967) (width 0.25) (layer "B.Cu") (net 32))
 (segment (start 92.9167 42.6862) (end 92.9167 43.9116) (width 0.25) (layer "F.Cu") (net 31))
 (segment (start 108.3433 42.6323) (end 107.0718 41.3608) (width 0.25) (layer "F.Cu") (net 31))
 (segment (start 88.6799 115.4401) (end 87.22 116.9) (width 0.25) (layer "F.Cu") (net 31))
 (segment (start 88.6799 63.1327) (end 88.6799 115.4401) (width 0.25) (layer "F.Cu") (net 31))
 (segment (start 94.2421 41.3608) (end 92.9167 42.6862) (width 0.25) (layer "F.Cu") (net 31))
 (segment (start 108.3433 43) (end 108.3433 42.6323) (width 0.25) (layer "F.Cu") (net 31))
 (segment (start 90.5424 61.2702) (end 88.6799 63.1327) (width 0.25) (layer "F.Cu") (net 31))
 (segment (start 90.5424 46.2859) (end 90.5424 61.2702) (width 0.25) (layer "F.Cu") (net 31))
 (segment (start 92.9167 43.9116) (end 90.5424 46.2859) (width 0.25) (layer "F.Cu") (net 31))
 (segment (start 109.52 43) (end 108.3433 43) (width 0.25) (layer "F.Cu") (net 31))
 (segment (start 107.0718 41.3608) (end 94.2421 41.3608) (width 0.25) (layer "F.Cu") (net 31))
 (segment (start 90.4 116.9) (end 90.4 62.4458) (width 0.25) (layer "F.Cu") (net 30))
 (via (at 90.4 62.4458) (size 0.8) (drill 0.4) (layers "F.Cu" "B.Cu") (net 30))
 (segment (start 106.98 43) (end 106.98 44.1767) (width 0.25) (layer "B.Cu") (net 30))
 (segment (start 106.7035 44.1767) (end 90.4 60.4802) (width 0.25) (layer "B.Cu") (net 30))
 (segment (start 90.4 60.4802) (end 90.4 62.4458) (width 0.25) (layer "B.Cu") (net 30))
 (segment (start 106.98 44.1767) (end 106.7035 44.1767) (width 0.25) (layer "B.Cu") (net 30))
 (segment (start 93.0224 45.4343) (end 93.0224 116.3424) (width 0.25) (layer "F.Cu") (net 26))
 (segment (start 94.28 43) (end 94.28 44.1767) (width 0.25) (layer "F.Cu") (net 26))
 (segment (start 93.0224 116.3424) (end 93.58 116.9) (width 0.25) (layer "F.Cu") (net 26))
 (segment (start 94.28 44.1767) (end 93.0224 45.4343) (width 0.25) (layer "F.Cu") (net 26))
 (segment (start 128.56 116.9) (end 128.56 111.5896) (width 0.25) (layer "F.Cu") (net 16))
 (segment (start 128.56 111.5896) (end 117.16 100.1896) (width 0.25) (layer "F.Cu") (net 16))
 (segment (start 117.16 100.1896) (end 117.16 60.8) (width 0.25) (layer "F.Cu") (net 16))
 (segment (start 131.74 116.9) (end 131.74 112.4753) (width 0.25) (layer "F.Cu") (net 17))
 (segment (start 131.74 112.4753) (end 119.7 100.4353) (width 0.25) (layer "F.Cu") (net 17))
 (segment (start 119.7 100.4353) (end 119.7 60.8) (width 0.25) (layer "F.Cu") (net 17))
 (segment (start 110.7019 42.5065) (end 110.7019 43.5705) (width 0.25) (layer "F.Cu") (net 28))
 (segment (start 106.4778 44.1767) (end 105.71 43.4089) (width 0.25) (layer "F.Cu") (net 28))
 (segment (start 84.04 116.9) (end 84.04 113.1424) (width 0.25) (layer "F.Cu") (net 28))
 (segment (start 110.7019 43.5705) (end 110.0957 44.1767) (width 0.25) (layer "F.Cu") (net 28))
 (segment (start 110.0957 44.1767) (end 106.4778 44.1767) (width 0.25) (layer "F.Cu") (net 28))
 (segment (start 109.1016 40.9062) (end 110.7019 42.5065) (width 0.25) (layer "F.Cu") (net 28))
 (segment (start 84.04 113.1424) (end 88.1565 109.0259) (width 0.25) (layer "F.Cu") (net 28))
 (segment (start 87.9997 61.6731) (end 87.9997 42.4871) (width 0.25) (layer "F.Cu") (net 28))
 (segment (start 100.5367 42.6322) (end 100.5367 43) (width 0.25) (layer "F.Cu") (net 28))
 (segment (start 88.1565 109.0259) (end 88.1565 61.8299) (width 0.25) (layer "F.Cu") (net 28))
 (segment (start 101.3456 41.8233) (end 100.5367 42.6322) (width 0.25) (layer "F.Cu") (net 28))
 (segment (start 87.9997 42.4871) (end 89.5806 40.9062) (width 0.25) (layer "F.Cu") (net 28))
 (segment (start 89.5806 40.9062) (end 109.1016 40.9062) (width 0.25) (layer "F.Cu") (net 28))
 (segment (start 105.71 43.4089) (end 105.71 42.5178) (width 0.25) (layer "F.Cu") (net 28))
 (segment (start 99.36 43) (end 100.5367 43) (width 0.25) (layer "F.Cu") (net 28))
 (segment (start 88.1565 61.8299) (end 87.9997 61.6731) (width 0.25) (layer "F.Cu") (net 28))
 (segment (start 105.0155 41.8233) (end 101.3456 41.8233) (width 0.25) (layer "F.Cu") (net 28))
 (segment (start 105.71 42.5178) (end 105.0155 41.8233) (width 0.25) (layer "F.Cu") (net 28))
 (segment (start 78.522 116.058) (end 77.68 116.9) (width 0.25) (layer "F.Cu") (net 21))
 (segment (start 133.0233 49.5991) (end 122.2142 38.79) (width 0.25) (layer "F.Cu") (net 21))
 (segment (start 86.11 36.9) (end 86.11 38.0267) (width 0.25) (layer "F.Cu") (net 21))
 (segment (start 133.0233 54.3) (end 133.0233 49.5991) (width 0.25) (layer "F.Cu") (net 21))
 (segment (start 134.1 54.3) (end 133.0233 54.3) (width 0.25) (layer "F.Cu") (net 21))
 (segment (start 86.8733 38.79) (end 85.4701 40.1932) (width 0.25) (layer "F.Cu") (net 21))
 (segment (start 122.2142 38.79) (end 86.8733 38.79) (width 0.25) (layer "F.Cu") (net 21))
 (segment (start 85.4701 40.1932) (end 85.4701 74.118) (width 0.25) (layer "F.Cu") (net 21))
 (segment (start 78.522 97.5122) (end 78.522 116.058) (width 0.25) (layer "F.Cu") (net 21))
 (segment (start 85.5303 90.5039) (end 78.522 97.5122) (width 0.25) (layer "F.Cu") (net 21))
 (segment (start 85.4701 74.118) (end 85.5303 74.1782) (width 0.25) (layer "F.Cu") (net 21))
 (segment (start 86.11 38.0267) (end 86.8733 38.79) (width 0.25) (layer "F.Cu") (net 21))
 (segment (start 85.5303 74.1782) (end 85.5303 90.5039) (width 0.25) (layer "F.Cu") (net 21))
 (segment (start 74.5 116.9) (end 77.68 116.9) (width 0.25) (layer "F.Cu") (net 21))
 (segment (start 113.2567 60.4322) (end 113.2567 60.8) (width 0.25) (layer "F.Cu") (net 6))
 (segment (start 138.1 116.9) (end 138.1 113.4081) (width 0.25) (layer "F.Cu") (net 6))
 (segment (start 112.08 60.8) (end 113.2567 60.8) (width 0.25) (layer "F.Cu") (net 6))
 (segment (start 104.44 43) (end 104.44 44.1767) (width 0.25) (layer "F.Cu") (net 6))
 (segment (start 120.2403 59.6233) (end 114.0656 59.6233) (width 0.25) (layer "F.Cu") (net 6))
 (segment (start 138.1 113.4081) (end 120.97 96.2781) (width 0.25) (layer "F.Cu") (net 6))
 (segment (start 114.0656 53.8023) (end 114.0656 59.6233) (width 0.25) (layer "F.Cu") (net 6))
 (segment (start 89.2 43) (end 89.2 59.6033) (width 0.25) (layer "F.Cu") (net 6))
 (segment (start 120.97 96.2781) (end 120.97 60.353) (width 0.25) (layer "F.Cu") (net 6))
 (segment (start 114.0656 59.6233) (end 113.2567 60.4322) (width 0.25) (layer "F.Cu") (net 6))
 (segment (start 89.2 59.6033) (end 89.22 59.6233) (width 0.25) (layer "F.Cu") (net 6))
 (segment (start 120.97 60.353) (end 120.2403 59.6233) (width 0.25) (layer "F.Cu") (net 6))
 (segment (start 141.28 116.9) (end 138.1 116.9) (width 0.25) (layer "F.Cu") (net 6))
 (segment (start 104.44 44.1767) (end 114.0656 53.8023) (width 0.25) (layer "F.Cu") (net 6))
 (segment (start 89.22 60.8) (end 89.22 59.6233) (width 0.25) (layer "F.Cu") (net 6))
 (segment (start 105.6167 42.6344) (end 108.4401 39.811) (width 0.25) (layer "B.Cu") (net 6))
 (segment (start 103.8517 43) (end 103.2633 43) (width 0.25) (layer "B.Cu") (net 6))
 (segment (start 131.389 39.811) (end 131.5 39.7) (width 0.25) (layer "B.Cu") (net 6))
 (segment (start 82.7567 42.6322) (end 82.7567 43) (width 0.25) (layer "B.Cu") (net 6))
 (segment (start 103.8517 43) (end 104.44 43) (width 0.25) (layer "B.Cu") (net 6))
 (segment (start 104.44 43) (end 105.6167 43) (width 0.25) (layer "B.Cu") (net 6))
 (segment (start 105.6167 43) (end 105.6167 42.6344) (width 0.25) (layer "B.Cu") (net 6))
 (segment (start 90.3767 43.3678) (end 90.3767 43) (width 0.25) (layer "B.Cu") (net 6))
 (segment (start 91.1856 44.1767) (end 90.3767 43.3678) (width 0.25) (layer "B.Cu") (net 6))
 (segment (start 81.58 43) (end 82.7567 43) (width 0.25) (layer "B.Cu") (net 6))
 (segment (start 103.2633 43) (end 103.2633 43.3678) (width 0.25) (layer "B.Cu") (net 6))
 (segment (start 103.2633 43.3678) (end 102.4544 44.1767) (width 0.25) (layer "B.Cu") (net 6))
 (segment (start 89.7884 43) (end 88.6117 41.8233) (width 0.25) (layer "B.Cu") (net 6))
 (segment (start 89.2 43) (end 89.7884 43) (width 0.25) (layer "B.Cu") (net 6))
 (segment (start 88.6117 41.8233) (end 83.5656 41.8233) (width 0.25) (layer "B.Cu") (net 6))
 (segment (start 108.4401 39.811) (end 131.389 39.811) (width 0.25) (layer "B.Cu") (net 6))
 (segment (start 83.5656 41.8233) (end 82.7567 42.6322) (width 0.25) (layer "B.Cu") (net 6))
 (segment (start 102.4544 44.1767) (end 91.1856 44.1767) (width 0.25) (layer "B.Cu") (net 6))
 (segment (start 89.7884 43) (end 90.3767 43) (width 0.25) (layer "B.Cu") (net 6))
 (segment (start 138 39.7) (end 131.5 39.7) (width 0.25) (layer "B.Cu") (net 6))
 (segment (start 103.12 45.3967) (end 101.9 44.1767) (width 0.25) (layer "F.Cu") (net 29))
 (segment (start 103.12 116.9) (end 103.12 45.3967) (width 0.25) (layer "F.Cu") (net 29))
 (segment (start 101.9 43) (end 101.9 44.1767) (width 0.25) (layer "F.Cu") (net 29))
 (segment (start 134.1 49.307) (end 123.8517 39.0587) (width 0.25) (layer "F.Cu") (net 27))
 (segment (start 96.82 43) (end 96.82 44.1767) (width 0.25) (layer "F.Cu") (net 27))
 (segment (start 134.1 53) (end 134.1 49.307) (width 0.25) (layer "F.Cu") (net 27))
 (segment (start 93.7491 55.6515) (end 93.7491 47.2476) (width 0.25) (layer "F.Cu") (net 27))
 (segment (start 80.86 111.8718) (end 87.421 105.3108) (width 0.25) (layer "F.Cu") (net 27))
 (segment (start 80.86 116.9) (end 80.86 111.8718) (width 0.25) (layer "F.Cu") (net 27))
 (segment (start 93.7491 47.2476) (end 96.82 44.1767) (width 0.25) (layer "F.Cu") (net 27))
 (segment (start 87.421 105.3108) (end 87.421 62.4301) (width 0.25) (layer "F.Cu") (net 27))
 (via (at 93.7491 55.6515) (size 0.8) (drill 0.4) (layers "F.Cu" "B.Cu") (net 27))
 (via (at 87.421 62.4301) (size 0.8) (drill 0.4) (layers "F.Cu" "B.Cu") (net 27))
 (via (at 123.8517 39.0587) (size 0.8) (drill 0.4) (layers "F.Cu" "B.Cu") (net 27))
 (segment (start 101.5766 39.0587) (end 123.8517 39.0587) (width 0.25) (layer "B.Cu") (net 27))
 (segment (start 97.9967 43) (end 97.9967 42.6386) (width 0.25) (layer "B.Cu") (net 27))
 (segment (start 87.95 60.3808) (end 87.95 61.9011) (width 0.25) (layer "B.Cu") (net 27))
 (segment (start 93.7491 55.6515) (end 92.6793 55.6515) (width 0.25) (layer "B.Cu") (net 27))
 (segment (start 96.82 43) (end 97.9967 43) (width 0.25) (layer "B.Cu") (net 27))
 (segment (start 87.95 61.9011) (end 87.421 62.4301) (width 0.25) (layer "B.Cu") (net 27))
 (segment (start 92.6793 55.6515) (end 87.95 60.3808) (width 0.25) (layer "B.Cu") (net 27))
 (segment (start 97.9967 42.6386) (end 101.5766 39.0587) (width 0.25) (layer "B.Cu") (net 27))
 (segment (start 79.04 43) (end 79.04 38.5767) (width 0.25) (layer "F.Cu") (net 20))
 (segment (start 79.04 38.5767) (end 78.49 38.0267) (width 0.25) (layer "F.Cu") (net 20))
 (segment (start 78.49 36.9) (end 78.49 38.0267) (width 0.25) (layer "F.Cu") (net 20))
 (segment (start 131.5 35.2) (end 100.349 35.2) (width 0.25) (layer "B.Cu") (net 25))
 (segment (start 138 35.2) (end 131.5 35.2) (width 0.25) (layer "B.Cu") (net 25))
 (segment (start 92.9167 42.6323) (end 92.9167 43) (width 0.25) (layer "B.Cu") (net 25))
 (segment (start 91.74 43) (end 92.9167 43) (width 0.25) (layer "B.Cu") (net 25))
 (segment (start 100.349 35.2) (end 92.9167 42.6323) (width 0.25) (layer "B.Cu") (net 25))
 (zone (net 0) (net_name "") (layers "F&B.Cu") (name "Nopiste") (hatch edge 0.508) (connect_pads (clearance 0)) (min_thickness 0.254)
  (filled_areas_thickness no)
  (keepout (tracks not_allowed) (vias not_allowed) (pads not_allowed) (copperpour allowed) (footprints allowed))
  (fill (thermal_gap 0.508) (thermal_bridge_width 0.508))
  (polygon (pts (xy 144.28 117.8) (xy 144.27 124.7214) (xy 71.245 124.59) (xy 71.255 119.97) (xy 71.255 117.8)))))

